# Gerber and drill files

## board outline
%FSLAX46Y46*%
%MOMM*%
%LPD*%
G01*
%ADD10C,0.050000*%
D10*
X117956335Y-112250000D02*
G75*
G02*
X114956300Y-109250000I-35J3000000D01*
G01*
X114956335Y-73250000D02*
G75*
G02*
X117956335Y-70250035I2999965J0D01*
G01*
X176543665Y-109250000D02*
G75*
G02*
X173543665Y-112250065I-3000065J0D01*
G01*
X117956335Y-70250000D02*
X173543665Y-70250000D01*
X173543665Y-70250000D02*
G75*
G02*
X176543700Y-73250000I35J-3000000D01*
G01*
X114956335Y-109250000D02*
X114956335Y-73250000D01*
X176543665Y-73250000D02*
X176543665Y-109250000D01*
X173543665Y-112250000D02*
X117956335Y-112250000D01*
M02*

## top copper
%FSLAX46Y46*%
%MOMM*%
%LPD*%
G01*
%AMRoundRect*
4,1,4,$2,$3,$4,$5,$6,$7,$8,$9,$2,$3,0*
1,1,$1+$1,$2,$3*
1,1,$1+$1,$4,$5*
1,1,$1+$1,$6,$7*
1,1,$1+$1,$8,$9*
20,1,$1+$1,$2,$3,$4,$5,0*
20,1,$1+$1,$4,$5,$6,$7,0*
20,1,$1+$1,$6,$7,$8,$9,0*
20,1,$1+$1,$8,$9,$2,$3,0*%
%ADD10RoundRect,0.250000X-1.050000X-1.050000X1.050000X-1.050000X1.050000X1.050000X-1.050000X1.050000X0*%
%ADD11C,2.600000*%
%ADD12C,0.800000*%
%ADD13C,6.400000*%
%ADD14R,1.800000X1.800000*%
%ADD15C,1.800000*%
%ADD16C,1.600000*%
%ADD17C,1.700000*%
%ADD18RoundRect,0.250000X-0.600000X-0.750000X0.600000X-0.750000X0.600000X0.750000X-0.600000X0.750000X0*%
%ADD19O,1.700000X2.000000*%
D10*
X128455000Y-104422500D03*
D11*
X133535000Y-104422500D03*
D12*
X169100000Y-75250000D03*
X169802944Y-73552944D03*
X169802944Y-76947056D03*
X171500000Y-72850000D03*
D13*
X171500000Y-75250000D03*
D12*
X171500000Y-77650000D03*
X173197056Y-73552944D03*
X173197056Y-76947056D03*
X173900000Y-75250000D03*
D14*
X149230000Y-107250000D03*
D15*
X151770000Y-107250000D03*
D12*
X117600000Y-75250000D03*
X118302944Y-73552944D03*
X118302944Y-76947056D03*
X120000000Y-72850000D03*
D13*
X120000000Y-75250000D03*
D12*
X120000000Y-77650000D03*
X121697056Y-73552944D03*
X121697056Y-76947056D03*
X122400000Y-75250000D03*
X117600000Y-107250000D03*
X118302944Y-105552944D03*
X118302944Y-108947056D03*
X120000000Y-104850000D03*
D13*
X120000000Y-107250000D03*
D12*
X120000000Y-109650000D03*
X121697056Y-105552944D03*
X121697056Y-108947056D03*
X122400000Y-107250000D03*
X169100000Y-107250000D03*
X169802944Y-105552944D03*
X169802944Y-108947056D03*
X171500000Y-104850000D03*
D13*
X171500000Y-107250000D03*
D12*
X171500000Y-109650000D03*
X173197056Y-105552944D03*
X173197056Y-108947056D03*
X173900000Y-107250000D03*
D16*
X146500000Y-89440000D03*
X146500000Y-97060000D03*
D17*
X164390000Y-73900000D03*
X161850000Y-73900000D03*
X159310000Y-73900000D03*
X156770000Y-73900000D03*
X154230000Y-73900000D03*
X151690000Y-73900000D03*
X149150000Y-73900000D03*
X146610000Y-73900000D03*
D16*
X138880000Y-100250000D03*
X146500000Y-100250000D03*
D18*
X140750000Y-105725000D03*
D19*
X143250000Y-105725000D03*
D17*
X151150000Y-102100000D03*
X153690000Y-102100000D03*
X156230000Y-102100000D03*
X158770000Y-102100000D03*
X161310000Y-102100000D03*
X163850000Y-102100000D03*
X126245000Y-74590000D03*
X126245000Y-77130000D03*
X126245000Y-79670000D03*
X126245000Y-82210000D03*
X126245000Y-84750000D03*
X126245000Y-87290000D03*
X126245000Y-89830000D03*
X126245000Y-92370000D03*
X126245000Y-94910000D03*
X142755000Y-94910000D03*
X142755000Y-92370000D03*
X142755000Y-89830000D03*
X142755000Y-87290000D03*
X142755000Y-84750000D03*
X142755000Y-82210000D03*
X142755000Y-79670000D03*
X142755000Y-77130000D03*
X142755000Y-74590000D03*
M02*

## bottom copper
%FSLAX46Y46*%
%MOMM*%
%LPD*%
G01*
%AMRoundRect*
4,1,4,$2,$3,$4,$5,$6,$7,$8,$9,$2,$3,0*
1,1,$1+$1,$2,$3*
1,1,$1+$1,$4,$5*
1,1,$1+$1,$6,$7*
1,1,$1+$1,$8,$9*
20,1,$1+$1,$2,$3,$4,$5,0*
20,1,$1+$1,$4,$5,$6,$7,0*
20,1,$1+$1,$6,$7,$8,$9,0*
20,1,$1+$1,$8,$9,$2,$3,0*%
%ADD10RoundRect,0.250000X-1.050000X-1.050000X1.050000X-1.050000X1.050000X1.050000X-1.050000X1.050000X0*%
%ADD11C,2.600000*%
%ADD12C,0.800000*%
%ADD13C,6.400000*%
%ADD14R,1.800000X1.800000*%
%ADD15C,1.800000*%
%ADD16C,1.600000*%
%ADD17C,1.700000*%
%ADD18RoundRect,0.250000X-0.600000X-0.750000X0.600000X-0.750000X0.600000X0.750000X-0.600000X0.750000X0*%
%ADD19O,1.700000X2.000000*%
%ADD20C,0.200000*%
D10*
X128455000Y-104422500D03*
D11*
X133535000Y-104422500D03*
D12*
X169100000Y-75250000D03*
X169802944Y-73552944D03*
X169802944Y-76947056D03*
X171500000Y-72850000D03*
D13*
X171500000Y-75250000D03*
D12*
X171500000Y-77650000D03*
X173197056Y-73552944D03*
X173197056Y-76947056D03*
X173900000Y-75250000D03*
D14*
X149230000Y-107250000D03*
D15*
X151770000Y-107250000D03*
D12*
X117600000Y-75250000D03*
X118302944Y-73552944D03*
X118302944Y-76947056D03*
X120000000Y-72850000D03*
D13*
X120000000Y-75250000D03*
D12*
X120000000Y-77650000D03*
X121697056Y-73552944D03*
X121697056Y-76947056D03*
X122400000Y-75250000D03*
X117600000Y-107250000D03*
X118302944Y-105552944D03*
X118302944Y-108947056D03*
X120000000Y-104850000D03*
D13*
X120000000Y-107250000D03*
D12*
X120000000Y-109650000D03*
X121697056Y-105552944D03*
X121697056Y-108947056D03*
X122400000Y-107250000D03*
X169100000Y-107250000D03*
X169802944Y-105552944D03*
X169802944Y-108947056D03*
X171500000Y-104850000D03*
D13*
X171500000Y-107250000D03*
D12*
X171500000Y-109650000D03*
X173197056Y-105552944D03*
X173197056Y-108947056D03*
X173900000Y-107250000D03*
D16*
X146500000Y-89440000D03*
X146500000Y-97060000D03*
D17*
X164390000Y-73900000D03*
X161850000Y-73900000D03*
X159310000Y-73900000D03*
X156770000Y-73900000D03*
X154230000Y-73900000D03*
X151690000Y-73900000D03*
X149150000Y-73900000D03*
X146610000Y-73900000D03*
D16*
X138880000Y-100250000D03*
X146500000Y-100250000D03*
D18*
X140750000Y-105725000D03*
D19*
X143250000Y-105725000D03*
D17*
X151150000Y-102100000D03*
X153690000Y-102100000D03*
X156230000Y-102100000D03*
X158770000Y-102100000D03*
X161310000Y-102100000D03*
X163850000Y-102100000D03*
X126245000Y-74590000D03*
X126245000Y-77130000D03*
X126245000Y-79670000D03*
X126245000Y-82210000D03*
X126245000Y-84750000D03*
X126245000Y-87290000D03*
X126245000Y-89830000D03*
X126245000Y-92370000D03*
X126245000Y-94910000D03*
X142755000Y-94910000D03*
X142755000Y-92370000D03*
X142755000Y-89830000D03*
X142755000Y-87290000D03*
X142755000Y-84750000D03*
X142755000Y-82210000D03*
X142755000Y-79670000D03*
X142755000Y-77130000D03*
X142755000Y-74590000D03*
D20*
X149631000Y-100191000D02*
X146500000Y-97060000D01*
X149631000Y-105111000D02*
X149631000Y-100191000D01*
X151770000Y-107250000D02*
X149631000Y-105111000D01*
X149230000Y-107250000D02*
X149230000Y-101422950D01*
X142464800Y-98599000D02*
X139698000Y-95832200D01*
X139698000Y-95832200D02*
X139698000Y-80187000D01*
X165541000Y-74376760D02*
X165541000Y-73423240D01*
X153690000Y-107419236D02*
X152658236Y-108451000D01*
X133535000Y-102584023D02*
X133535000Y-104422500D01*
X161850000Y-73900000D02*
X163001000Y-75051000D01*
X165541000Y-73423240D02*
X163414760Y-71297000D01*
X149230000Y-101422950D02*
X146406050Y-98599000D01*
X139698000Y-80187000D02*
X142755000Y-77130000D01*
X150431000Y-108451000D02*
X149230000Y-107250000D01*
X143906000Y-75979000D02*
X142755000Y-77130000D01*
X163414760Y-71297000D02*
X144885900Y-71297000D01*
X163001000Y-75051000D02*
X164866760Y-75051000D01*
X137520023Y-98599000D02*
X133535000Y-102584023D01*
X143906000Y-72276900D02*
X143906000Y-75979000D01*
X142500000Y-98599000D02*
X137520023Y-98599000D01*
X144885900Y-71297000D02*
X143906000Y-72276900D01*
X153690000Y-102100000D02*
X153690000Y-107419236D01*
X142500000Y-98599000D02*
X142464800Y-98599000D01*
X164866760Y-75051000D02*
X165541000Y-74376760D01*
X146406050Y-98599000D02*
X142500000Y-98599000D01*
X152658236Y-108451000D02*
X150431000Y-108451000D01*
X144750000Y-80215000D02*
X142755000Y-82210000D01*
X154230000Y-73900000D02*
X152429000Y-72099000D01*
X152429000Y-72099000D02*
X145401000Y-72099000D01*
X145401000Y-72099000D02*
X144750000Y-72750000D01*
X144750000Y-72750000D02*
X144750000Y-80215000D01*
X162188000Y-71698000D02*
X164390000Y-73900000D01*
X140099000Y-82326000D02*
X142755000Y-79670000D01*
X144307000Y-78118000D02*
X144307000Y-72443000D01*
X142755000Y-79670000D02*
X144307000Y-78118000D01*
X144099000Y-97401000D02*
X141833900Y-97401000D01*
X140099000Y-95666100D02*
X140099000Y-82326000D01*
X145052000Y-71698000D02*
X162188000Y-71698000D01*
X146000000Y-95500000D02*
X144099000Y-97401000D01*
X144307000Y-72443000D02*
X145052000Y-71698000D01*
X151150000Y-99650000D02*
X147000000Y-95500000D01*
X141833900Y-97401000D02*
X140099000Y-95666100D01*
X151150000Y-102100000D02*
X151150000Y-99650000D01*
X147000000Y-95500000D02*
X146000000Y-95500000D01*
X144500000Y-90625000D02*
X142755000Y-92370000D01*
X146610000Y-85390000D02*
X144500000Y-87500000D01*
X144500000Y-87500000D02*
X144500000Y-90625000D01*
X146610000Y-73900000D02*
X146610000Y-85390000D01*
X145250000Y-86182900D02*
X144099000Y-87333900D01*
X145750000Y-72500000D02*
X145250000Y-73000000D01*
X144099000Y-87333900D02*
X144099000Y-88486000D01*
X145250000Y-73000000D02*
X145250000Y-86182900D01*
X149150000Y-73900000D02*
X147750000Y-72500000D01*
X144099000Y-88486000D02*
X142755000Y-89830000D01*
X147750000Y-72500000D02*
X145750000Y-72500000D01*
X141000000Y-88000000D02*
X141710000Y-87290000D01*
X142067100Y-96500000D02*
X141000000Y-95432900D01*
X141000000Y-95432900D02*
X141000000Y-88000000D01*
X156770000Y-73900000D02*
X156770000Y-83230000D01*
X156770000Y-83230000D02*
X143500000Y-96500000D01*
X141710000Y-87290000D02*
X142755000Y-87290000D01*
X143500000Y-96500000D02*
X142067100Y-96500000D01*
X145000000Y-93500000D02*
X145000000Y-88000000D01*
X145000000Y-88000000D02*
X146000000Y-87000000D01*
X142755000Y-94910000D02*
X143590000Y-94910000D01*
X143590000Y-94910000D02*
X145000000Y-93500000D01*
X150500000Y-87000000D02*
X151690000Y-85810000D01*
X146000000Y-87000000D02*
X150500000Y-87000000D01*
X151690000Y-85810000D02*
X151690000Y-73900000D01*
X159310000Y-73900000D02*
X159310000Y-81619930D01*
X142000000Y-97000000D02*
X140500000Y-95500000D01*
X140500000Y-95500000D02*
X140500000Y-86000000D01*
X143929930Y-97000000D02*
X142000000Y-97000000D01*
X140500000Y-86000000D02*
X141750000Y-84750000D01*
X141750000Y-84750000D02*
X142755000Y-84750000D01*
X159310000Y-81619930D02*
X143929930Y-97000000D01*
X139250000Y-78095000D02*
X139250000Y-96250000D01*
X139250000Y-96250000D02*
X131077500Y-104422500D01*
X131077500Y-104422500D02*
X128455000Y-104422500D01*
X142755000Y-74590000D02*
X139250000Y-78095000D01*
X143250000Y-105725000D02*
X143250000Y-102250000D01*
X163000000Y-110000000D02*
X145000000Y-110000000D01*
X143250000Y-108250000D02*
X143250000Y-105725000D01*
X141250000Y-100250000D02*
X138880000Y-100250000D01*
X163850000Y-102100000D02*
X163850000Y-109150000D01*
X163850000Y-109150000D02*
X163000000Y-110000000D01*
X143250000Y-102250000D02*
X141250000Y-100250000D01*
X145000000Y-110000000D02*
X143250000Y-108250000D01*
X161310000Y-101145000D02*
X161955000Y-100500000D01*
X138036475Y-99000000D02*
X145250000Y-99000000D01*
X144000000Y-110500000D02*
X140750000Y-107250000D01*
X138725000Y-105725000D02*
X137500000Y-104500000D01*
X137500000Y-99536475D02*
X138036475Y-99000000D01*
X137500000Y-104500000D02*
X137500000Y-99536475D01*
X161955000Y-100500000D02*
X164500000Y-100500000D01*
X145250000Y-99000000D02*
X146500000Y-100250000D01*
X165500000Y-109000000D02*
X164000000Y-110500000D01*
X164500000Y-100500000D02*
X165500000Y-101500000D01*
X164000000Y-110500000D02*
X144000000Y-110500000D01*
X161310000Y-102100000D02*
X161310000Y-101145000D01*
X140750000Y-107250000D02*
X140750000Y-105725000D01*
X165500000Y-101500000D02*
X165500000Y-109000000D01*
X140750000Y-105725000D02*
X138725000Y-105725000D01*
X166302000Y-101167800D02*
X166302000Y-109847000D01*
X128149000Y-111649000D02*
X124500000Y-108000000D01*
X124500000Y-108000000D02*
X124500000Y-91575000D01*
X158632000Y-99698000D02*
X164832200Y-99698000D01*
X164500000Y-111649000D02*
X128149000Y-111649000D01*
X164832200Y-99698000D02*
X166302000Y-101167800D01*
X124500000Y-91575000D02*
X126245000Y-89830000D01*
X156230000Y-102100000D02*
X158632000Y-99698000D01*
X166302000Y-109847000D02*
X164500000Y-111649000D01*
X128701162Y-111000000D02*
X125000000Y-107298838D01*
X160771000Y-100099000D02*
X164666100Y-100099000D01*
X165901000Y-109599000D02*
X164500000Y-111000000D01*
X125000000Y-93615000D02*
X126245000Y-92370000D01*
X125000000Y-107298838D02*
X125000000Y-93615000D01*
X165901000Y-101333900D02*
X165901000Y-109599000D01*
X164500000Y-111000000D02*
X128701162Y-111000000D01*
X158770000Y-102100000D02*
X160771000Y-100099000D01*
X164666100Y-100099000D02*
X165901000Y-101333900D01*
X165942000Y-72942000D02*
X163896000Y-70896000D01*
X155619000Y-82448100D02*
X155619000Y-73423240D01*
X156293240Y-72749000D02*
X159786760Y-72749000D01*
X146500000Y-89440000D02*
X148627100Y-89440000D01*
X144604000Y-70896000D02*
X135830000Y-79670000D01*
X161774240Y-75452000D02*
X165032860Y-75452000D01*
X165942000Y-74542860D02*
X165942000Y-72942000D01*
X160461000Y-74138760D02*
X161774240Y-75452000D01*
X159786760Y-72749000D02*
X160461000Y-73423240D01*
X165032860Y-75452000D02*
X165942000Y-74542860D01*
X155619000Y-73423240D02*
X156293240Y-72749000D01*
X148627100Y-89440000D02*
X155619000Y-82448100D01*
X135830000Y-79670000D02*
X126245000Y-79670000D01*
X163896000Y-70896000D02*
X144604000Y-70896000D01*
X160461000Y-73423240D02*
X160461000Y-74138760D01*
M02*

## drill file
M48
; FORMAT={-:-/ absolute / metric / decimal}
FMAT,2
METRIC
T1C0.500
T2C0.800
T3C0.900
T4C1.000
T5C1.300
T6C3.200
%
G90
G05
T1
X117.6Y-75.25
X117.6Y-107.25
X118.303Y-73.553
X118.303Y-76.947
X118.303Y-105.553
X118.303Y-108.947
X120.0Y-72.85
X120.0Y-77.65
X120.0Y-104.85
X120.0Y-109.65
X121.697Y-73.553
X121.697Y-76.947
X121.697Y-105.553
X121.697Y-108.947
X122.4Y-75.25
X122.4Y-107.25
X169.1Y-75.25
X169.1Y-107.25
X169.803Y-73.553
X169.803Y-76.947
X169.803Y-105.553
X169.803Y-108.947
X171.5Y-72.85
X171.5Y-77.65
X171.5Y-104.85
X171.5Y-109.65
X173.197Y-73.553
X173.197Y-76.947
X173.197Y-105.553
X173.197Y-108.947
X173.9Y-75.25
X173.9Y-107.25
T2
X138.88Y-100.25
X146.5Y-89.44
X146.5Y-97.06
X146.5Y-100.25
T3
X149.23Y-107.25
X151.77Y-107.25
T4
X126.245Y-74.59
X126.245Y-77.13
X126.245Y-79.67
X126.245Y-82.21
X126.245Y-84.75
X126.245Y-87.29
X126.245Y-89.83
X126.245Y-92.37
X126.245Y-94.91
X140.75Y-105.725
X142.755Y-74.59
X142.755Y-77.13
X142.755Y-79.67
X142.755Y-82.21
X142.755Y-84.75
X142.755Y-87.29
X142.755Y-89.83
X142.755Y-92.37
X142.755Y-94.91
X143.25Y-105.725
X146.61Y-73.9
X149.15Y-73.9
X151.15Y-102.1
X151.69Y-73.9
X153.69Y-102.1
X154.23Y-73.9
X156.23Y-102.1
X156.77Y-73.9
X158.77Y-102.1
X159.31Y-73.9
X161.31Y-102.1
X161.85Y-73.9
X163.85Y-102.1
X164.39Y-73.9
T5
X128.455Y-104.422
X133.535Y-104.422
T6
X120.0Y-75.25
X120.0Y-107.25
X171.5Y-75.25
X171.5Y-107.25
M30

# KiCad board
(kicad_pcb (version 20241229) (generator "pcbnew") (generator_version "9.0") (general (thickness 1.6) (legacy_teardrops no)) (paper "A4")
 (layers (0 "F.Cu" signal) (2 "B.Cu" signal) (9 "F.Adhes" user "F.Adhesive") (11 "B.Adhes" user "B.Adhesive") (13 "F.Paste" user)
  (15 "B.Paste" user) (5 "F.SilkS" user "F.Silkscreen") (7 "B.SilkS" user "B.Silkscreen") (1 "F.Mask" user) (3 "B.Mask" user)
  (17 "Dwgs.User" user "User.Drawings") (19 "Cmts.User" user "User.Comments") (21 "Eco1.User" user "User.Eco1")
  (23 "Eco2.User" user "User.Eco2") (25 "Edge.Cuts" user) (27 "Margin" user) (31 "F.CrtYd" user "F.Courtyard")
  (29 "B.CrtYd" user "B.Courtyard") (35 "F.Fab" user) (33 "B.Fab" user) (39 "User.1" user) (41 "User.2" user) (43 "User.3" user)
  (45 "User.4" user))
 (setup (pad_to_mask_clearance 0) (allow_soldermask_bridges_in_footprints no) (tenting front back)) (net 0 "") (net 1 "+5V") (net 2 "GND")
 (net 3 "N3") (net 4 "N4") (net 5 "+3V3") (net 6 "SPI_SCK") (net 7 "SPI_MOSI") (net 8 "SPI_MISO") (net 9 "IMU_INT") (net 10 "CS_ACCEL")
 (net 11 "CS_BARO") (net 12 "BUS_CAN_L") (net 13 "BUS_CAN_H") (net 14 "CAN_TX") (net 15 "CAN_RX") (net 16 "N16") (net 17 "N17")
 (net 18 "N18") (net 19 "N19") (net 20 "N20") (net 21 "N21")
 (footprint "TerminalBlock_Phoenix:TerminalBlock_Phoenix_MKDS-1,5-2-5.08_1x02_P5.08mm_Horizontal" (layer "F.Cu") (at 128.455 104.4225)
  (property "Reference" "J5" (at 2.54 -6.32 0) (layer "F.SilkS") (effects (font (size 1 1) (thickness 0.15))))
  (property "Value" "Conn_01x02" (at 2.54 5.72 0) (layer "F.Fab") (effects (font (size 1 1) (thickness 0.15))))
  (pad "1" thru_hole roundrect (at 0 0) (size 2.6 2.6) (drill 1.3) (layers "*.Cu" "*.Mask") (remove_unused_layers no)
   (roundrect_rratio 0.096154) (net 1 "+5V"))
  (pad "2" thru_hole circle (at 5.08 0) (size 2.6 2.6) (drill 1.3) (layers "*.Cu" "*.Mask") (remove_unused_layers no) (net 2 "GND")))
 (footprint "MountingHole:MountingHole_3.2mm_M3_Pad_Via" (layer "F.Cu") (at 171.5 75.25)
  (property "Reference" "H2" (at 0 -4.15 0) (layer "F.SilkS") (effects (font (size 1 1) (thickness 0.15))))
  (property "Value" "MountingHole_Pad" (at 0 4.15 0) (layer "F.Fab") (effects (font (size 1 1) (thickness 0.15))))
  (pad "1" thru_hole circle (at -2.4 0) (size 0.8 0.8) (drill 0.5) (layers "*.Cu" "*.Mask") (remove_unused_layers no) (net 2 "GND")
   (zone_connect 2))
  (pad "1" thru_hole circle (at -1.697056 -1.697056) (size 0.8 0.8) (drill 0.5) (layers "*.Cu" "*.Mask") (remove_unused_layers no)
   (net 2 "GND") (zone_connect 2))
  (pad "1" thru_hole circle (at -1.697056 1.697056) (size 0.8 0.8) (drill 0.5) (layers "*.Cu" "*.Mask") (remove_unused_layers no)
   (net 2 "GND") (zone_connect 2))
  (pad "1" thru_hole circle (at 0 -2.4) (size 0.8 0.8) (drill 0.5) (layers "*.Cu" "*.Mask") (remove_unused_layers no) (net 2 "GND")
   (zone_connect 2))
  (pad "1" thru_hole circle (at 0 0) (size 6.4 6.4) (drill 3.2) (layers "*.Cu" "*.Mask") (remove_unused_layers no) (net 2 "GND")
   (zone_connect 2))
  (pad "1" thru_hole circle (at 0 2.4) (size 0.8 0.8) (drill 0.5) (layers "*.Cu" "*.Mask") (remove_unused_layers no) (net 2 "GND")
   (zone_connect 2))
  (pad "1" thru_hole circle (at 1.697056 -1.697056) (size 0.8 0.8) (drill 0.5) (layers "*.Cu" "*.Mask") (remove_unused_layers no)
   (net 2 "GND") (zone_connect 2))
  (pad "1" thru_hole circle (at 1.697056 1.697056) (size 0.8 0.8) (drill 0.5) (layers "*.Cu" "*.Mask") (remove_unused_layers no)
   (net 2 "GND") (zone_connect 2))
  (pad "1" thru_hole circle (at 2.4 0) (size 0.8 0.8) (drill 0.5) (layers "*.Cu" "*.Mask") (remove_unused_layers no) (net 2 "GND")
   (zone_connect 2)))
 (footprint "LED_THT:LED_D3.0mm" (layer "F.Cu") (at 149.23 107.25)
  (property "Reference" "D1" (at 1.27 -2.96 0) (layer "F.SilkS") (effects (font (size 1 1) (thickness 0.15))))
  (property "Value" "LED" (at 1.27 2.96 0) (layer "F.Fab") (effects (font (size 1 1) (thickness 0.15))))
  (pad "1" thru_hole rect (at 0 0) (size 1.8 1.8) (drill 0.9) (layers "*.Cu" "*.Mask") (remove_unused_layers no) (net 2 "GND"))
  (pad "2" thru_hole circle (at 2.54 0) (size 1.8 1.8) (drill 0.9) (layers "*.Cu" "*.Mask") (remove_unused_layers no) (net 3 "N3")))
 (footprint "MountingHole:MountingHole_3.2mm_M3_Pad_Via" (layer "F.Cu") (at 120 75.25)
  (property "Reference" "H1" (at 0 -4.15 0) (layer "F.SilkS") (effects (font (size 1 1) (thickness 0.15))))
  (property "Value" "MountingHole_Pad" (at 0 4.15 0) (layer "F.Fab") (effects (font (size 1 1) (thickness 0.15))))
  (pad "1" thru_hole circle (at -2.4 0) (size 0.8 0.8) (drill 0.5) (layers "*.Cu" "*.Mask") (remove_unused_layers no) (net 2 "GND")
   (zone_connect 2))
  (pad "1" thru_hole circle (at -1.697056 -1.697056) (size 0.8 0.8) (drill 0.5) (layers "*.Cu" "*.Mask") (remove_unused_layers no)
   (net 2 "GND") (zone_connect 2))
  (pad "1" thru_hole circle (at -1.697056 1.697056) (size 0.8 0.8) (drill 0.5) (layers "*.Cu" "*.Mask") (remove_unused_layers no)
   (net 2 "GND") (zone_connect 2))
  (pad "1" thru_hole circle (at 0 -2.4) (size 0.8 0.8) (drill 0.5) (layers "*.Cu" "*.Mask") (remove_unused_layers no) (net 2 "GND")
   (zone_connect 2))
  (pad "1" thru_hole circle (at 0 0) (size 6.4 6.4) (drill 3.2) (layers "*.Cu" "*.Mask") (remove_unused_layers no) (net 2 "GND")
   (zone_connect 2))
  (pad "1" thru_hole circle (at 0 2.4) (size 0.8 0.8) (drill 0.5) (layers "*.Cu" "*.Mask") (remove_unused_layers no) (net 2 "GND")
   (zone_connect 2))
  (pad "1" thru_hole circle (at 1.697056 -1.697056) (size 0.8 0.8) (drill 0.5) (layers "*.Cu" "*.Mask") (remove_unused_layers no)
   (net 2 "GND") (zone_connect 2))
  (pad "1" thru_hole circle (at 1.697056 1.697056) (size 0.8 0.8) (drill 0.5) (layers "*.Cu" "*.Mask") (remove_unused_layers no)
   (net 2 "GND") (zone_connect 2))
  (pad "1" thru_hole circle (at 2.4 0) (size 0.8 0.8) (drill 0.5) (layers "*.Cu" "*.Mask") (remove_unused_layers no) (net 2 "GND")
   (zone_connect 2)))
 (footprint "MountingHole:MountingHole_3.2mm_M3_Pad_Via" (layer "F.Cu") (at 120 107.25)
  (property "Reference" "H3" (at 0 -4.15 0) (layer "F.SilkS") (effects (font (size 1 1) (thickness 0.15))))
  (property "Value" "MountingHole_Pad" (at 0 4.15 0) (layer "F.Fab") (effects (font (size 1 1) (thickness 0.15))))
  (pad "1" thru_hole circle (at -2.4 0) (size 0.8 0.8) (drill 0.5) (layers "*.Cu" "*.Mask") (remove_unused_layers no) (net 2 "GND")
   (zone_connect 2))
  (pad "1" thru_hole circle (at -1.697056 -1.697056) (size 0.8 0.8) (drill 0.5) (layers "*.Cu" "*.Mask") (remove_unused_layers no)
   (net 2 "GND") (zone_connect 2))
  (pad "1" thru_hole circle (at -1.697056 1.697056) (size 0.8 0.8) (drill 0.5) (layers "*.Cu" "*.Mask") (remove_unused_layers no)
   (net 2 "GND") (zone_connect 2))
  (pad "1" thru_hole circle (at 0 -2.4) (size 0.8 0.8) (drill 0.5) (layers "*.Cu" "*.Mask") (remove_unused_layers no) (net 2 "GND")
   (zone_connect 2))
  (pad "1" thru_hole circle (at 0 0) (size 6.4 6.4) (drill 3.2) (layers "*.Cu" "*.Mask") (remove_unused_layers no) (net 2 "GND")
   (zone_connect 2))
  (pad "1" thru_hole circle (at 0 2.4) (size 0.8 0.8) (drill 0.5) (layers "*.Cu" "*.Mask") (remove_unused_layers no) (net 2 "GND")
   (zone_connect 2))
  (pad "1" thru_hole circle (at 1.697056 -1.697056) (size 0.8 0.8) (drill 0.5) (layers "*.Cu" "*.Mask") (remove_unused_layers no)
   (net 2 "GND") (zone_connect 2))
  (pad "1" thru_hole circle (at 1.697056 1.697056) (size 0.8 0.8) (drill 0.5) (layers "*.Cu" "*.Mask") (remove_unused_layers no)
   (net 2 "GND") (zone_connect 2))
  (pad "1" thru_hole circle (at 2.4 0) (size 0.8 0.8) (drill 0.5) (layers "*.Cu" "*.Mask") (remove_unused_layers no) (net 2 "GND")
   (zone_connect 2)))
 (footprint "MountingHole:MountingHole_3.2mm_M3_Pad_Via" (layer "F.Cu") (at 171.5 107.25)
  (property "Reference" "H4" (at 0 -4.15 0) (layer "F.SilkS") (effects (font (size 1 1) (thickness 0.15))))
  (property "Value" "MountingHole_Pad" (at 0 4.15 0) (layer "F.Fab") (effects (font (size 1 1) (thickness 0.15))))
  (pad "1" thru_hole circle (at -2.4 0) (size 0.8 0.8) (drill 0.5) (layers "*.Cu" "*.Mask") (remove_unused_layers no) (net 2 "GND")
   (zone_connect 2))
  (pad "1" thru_hole circle (at -1.697056 -1.697056) (size 0.8 0.8) (drill 0.5) (layers "*.Cu" "*.Mask") (remove_unused_layers no)
   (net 2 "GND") (zone_connect 2))
  (pad "1" thru_hole circle (at -1.697056 1.697056) (size 0.8 0.8) (drill 0.5) (layers "*.Cu" "*.Mask") (remove_unused_layers no)
   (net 2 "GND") (zone_connect 2))
  (pad "1" thru_hole circle (at 0 -2.4) (size 0.8 0.8) (drill 0.5) (layers "*.Cu" "*.Mask") (remove_unused_layers no) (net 2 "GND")
   (zone_connect 2))
  (pad "1" thru_hole circle (at 0 0) (size 6.4 6.4) (drill 3.2) (layers "*.Cu" "*.Mask") (remove_unused_layers no) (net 2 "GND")
   (zone_connect 2))
  (pad "1" thru_hole circle (at 0 2.4) (size 0.8 0.8) (drill 0.5) (layers "*.Cu" "*.Mask") (remove_unused_layers no) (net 2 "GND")
   (zone_connect 2))
  (pad "1" thru_hole circle (at 1.697056 -1.697056) (size 0.8 0.8) (drill 0.5) (layers "*.Cu" "*.Mask") (remove_unused_layers no)
   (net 2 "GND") (zone_connect 2))
  (pad "1" thru_hole circle (at 1.697056 1.697056) (size 0.8 0.8) (drill 0.5) (layers "*.Cu" "*.Mask") (remove_unused_layers no)
   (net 2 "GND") (zone_connect 2))
  (pad "1" thru_hole circle (at 2.4 0) (size 0.8 0.8) (drill 0.5) (layers "*.Cu" "*.Mask") (remove_unused_layers no) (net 2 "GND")
   (zone_connect 2)))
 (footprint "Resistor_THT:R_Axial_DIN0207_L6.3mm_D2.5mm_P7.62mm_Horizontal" (layer "F.Cu") (at 146.5 89.44 -90)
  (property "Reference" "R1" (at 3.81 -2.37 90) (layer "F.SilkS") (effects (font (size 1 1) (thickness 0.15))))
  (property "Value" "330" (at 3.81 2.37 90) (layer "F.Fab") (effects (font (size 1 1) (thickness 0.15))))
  (pad "1" thru_hole circle (at 0 0 270) (size 1.6 1.6) (drill 0.8) (layers "*.Cu" "*.Mask") (remove_unused_layers no) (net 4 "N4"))
  (pad "2" thru_hole circle (at 7.62 0 270) (size 1.6 1.6) (drill 0.8) (layers "*.Cu" "*.Mask") (remove_unused_layers no) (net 3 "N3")))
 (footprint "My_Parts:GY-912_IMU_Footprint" (layer "F.Cu") (at 155.5 80.25 -90)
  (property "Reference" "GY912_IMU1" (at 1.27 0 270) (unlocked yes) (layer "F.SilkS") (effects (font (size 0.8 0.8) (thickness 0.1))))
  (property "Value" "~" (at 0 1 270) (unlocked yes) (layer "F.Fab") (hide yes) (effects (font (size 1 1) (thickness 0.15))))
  (pad "1" thru_hole circle (at -6.35 -8.89 270) (size 1.7 1.7) (drill 1) (layers "*.Cu" "*.Mask") (remove_unused_layers no) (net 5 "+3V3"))
  (pad "2" thru_hole circle (at -6.35 -6.35 270) (size 1.7 1.7) (drill 1) (layers "*.Cu" "*.Mask") (remove_unused_layers no) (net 2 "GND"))
  (pad "3" thru_hole circle (at -6.35 -3.81 270) (size 1.7 1.7) (drill 1) (layers "*.Cu" "*.Mask") (remove_unused_layers no)
   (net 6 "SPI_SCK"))
  (pad "4" thru_hole circle (at -6.35 -1.27 270) (size 1.7 1.7) (drill 1) (layers "*.Cu" "*.Mask") (remove_unused_layers no)
   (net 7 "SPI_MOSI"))
  (pad "5" thru_hole circle (at -6.35 1.27 270) (size 1.7 1.7) (drill 1) (layers "*.Cu" "*.Mask") (remove_unused_layers no)
   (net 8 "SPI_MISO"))
  (pad "6" thru_hole circle (at -6.35 3.81 270) (size 1.7 1.7) (drill 1) (layers "*.Cu" "*.Mask") (remove_unused_layers no)
   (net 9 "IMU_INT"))
  (pad "7" thru_hole circle (at -6.35 6.35 270) (size 1.7 1.7) (drill 1) (layers "*.Cu" "*.Mask") (remove_unused_layers no)
   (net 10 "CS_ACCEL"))
  (pad "8" thru_hole circle (at -6.35 8.89 270) (size 1.7 1.7) (drill 1) (layers "*.Cu" "*.Mask") (remove_unused_layers no)
   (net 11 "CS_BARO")))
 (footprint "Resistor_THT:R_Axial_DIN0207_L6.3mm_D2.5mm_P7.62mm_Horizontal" (layer "F.Cu") (at 138.88 100.25)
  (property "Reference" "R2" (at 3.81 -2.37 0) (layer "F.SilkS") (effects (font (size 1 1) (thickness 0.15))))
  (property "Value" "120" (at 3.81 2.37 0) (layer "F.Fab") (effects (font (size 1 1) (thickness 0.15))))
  (pad "1" thru_hole circle (at 0 0) (size 1.6 1.6) (drill 0.8) (layers "*.Cu" "*.Mask") (remove_unused_layers no) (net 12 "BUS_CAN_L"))
  (pad "2" thru_hole circle (at 7.62 0) (size 1.6 1.6) (drill 0.8) (layers "*.Cu" "*.Mask") (remove_unused_layers no) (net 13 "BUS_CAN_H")))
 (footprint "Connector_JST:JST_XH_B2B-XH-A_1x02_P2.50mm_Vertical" (layer "F.Cu") (at 140.75 105.725)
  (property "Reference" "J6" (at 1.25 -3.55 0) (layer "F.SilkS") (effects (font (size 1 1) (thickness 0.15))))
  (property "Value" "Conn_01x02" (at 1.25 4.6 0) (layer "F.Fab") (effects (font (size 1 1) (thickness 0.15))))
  (pad "1" thru_hole roundrect (at 0 0) (size 1.7 2) (drill 1) (layers "*.Cu" "*.Mask") (remove_unused_layers no)
   (roundrect_rratio 0.147059) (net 13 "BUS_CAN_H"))
  (pad "2" thru_hole oval (at 2.5 0) (size 1.7 2) (drill 1) (layers "*.Cu" "*.Mask") (remove_unused_layers no) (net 12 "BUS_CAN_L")))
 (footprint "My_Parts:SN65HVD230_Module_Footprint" (layer "F.Cu") (at 157.5 95.75 90)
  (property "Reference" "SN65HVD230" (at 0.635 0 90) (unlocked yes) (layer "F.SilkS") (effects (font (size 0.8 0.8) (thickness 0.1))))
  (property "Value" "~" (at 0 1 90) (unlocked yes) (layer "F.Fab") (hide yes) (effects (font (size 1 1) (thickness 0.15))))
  (pad "1" thru_hole circle (at -6.35 -6.35 90) (size 1.7 1.7) (drill 1) (layers "*.Cu" "*.Mask") (remove_unused_layers no) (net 5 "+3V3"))
  (pad "2" thru_hole circle (at -6.35 -3.81 90) (size 1.7 1.7) (drill 1) (layers "*.Cu" "*.Mask") (remove_unused_layers no) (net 2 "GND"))
  (pad "3" thru_hole circle (at -6.35 -1.27 90) (size 1.7 1.7) (drill 1) (layers "*.Cu" "*.Mask") (remove_unused_layers no)
   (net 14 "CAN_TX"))
  (pad "4" thru_hole circle (at -6.35 1.27 90) (size 1.7 1.7) (drill 1) (layers "*.Cu" "*.Mask") (remove_unused_layers no) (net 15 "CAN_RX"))
  (pad "5" thru_hole circle (at -6.35 3.81 90) (size 1.7 1.7) (drill 1) (layers "*.Cu" "*.Mask") (remove_unused_layers no)
   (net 13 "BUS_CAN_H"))
  (pad "6" thru_hole circle (at -6.35 6.35 90) (size 1.7 1.7) (drill 1) (layers "*.Cu" "*.Mask") (remove_unused_layers no)
   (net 12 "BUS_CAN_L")))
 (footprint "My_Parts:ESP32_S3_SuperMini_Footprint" (layer "F.Cu") (at 134.5 84.75)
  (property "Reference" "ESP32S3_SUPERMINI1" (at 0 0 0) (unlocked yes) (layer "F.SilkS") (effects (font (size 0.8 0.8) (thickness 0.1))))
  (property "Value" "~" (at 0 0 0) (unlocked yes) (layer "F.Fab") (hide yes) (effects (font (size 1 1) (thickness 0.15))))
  (pad "1" thru_hole circle (at -8.255 -10.16) (size 1.7 1.7) (drill 1) (layers "*.Cu" "*.Mask") (remove_unused_layers no) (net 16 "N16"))
  (pad "2" thru_hole circle (at -8.255 -7.62) (size 1.7 1.7) (drill 1) (layers "*.Cu" "*.Mask") (remove_unused_layers no) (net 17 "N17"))
  (pad "3" thru_hole circle (at -8.255 -5.08) (size 1.7 1.7) (drill 1) (layers "*.Cu" "*.Mask") (remove_unused_layers no) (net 4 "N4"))
  (pad "4" thru_hole circle (at -8.255 -2.54) (size 1.7 1.7) (drill 1) (layers "*.Cu" "*.Mask") (remove_unused_layers no) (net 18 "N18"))
  (pad "5" thru_hole circle (at -8.255 0) (size 1.7 1.7) (drill 1) (layers "*.Cu" "*.Mask") (remove_unused_layers no) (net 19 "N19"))
  (pad "6" thru_hole circle (at -8.255 2.54) (size 1.7 1.7) (drill 1) (layers "*.Cu" "*.Mask") (remove_unused_layers no) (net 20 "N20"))
  (pad "7" thru_hole circle (at -8.255 5.08) (size 1.7 1.7) (drill 1) (layers "*.Cu" "*.Mask") (remove_unused_layers no) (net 14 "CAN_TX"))
  (pad "8" thru_hole circle (at -8.255 7.62) (size 1.7 1.7) (drill 1) (layers "*.Cu" "*.Mask") (remove_unused_layers no) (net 15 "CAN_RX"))
  (pad "9" thru_hole circle (at -8.255 10.16) (size 1.7 1.7) (drill 1) (layers "*.Cu" "*.Mask") (remove_unused_layers no) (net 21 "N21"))
  (pad "10" thru_hole circle (at 8.255 10.16) (size 1.7 1.7) (drill 1) (layers "*.Cu" "*.Mask") (remove_unused_layers no) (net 9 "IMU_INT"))
  (pad "11" thru_hole circle (at 8.255 7.62) (size 1.7 1.7) (drill 1) (layers "*.Cu" "*.Mask") (remove_unused_layers no) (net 11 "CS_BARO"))
  (pad "12" thru_hole circle (at 8.255 5.08) (size 1.7 1.7) (drill 1) (layers "*.Cu" "*.Mask") (remove_unused_layers no) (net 10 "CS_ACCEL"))
  (pad "13" thru_hole circle (at 8.255 2.54) (size 1.7 1.7) (drill 1) (layers "*.Cu" "*.Mask") (remove_unused_layers no) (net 7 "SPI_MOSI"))
  (pad "14" thru_hole circle (at 8.255 0) (size 1.7 1.7) (drill 1) (layers "*.Cu" "*.Mask") (remove_unused_layers no) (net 6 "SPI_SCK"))
  (pad "15" thru_hole circle (at 8.255 -2.54) (size 1.7 1.7) (drill 1) (layers "*.Cu" "*.Mask") (remove_unused_layers no) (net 8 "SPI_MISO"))
  (pad "16" thru_hole circle (at 8.255 -5.08) (size 1.7 1.7) (drill 1) (layers "*.Cu" "*.Mask") (remove_unused_layers no) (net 5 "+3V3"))
  (pad "17" thru_hole circle (at 8.255 -7.62) (size 1.7 1.7) (drill 1) (layers "*.Cu" "*.Mask") (remove_unused_layers no) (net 2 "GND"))
  (pad "18" thru_hole circle (at 8.255 -10.16) (size 1.7 1.7) (drill 1) (layers "*.Cu" "*.Mask") (remove_unused_layers no) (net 1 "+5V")))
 (gr_arc (start 117.956335 112.25) (mid 115.835015 111.37132) (end 114.956335 109.25) (stroke (width 0.05) (type default))
  (layer "Edge.Cuts"))
 (gr_arc (start 114.956335 73.25) (mid 115.835015 71.12868) (end 117.956335 70.25) (stroke (width 0.05) (type default)) (layer "Edge.Cuts"))
 (gr_arc (start 176.543665 109.25) (mid 175.664983 111.371308) (end 173.543665 112.25) (stroke (width 0.05) (type default))
  (layer "Edge.Cuts"))
 (gr_line (start 117.956335 70.25) (end 173.543665 70.25) (stroke (width 0.05) (type default)) (layer "Edge.Cuts"))
 (gr_arc (start 173.543665 70.25) (mid 175.664985 71.12868) (end 176.543665 73.25) (stroke (width 0.05) (type default)) (layer "Edge.Cuts"))
 (gr_line (start 114.956335 109.25) (end 114.956335 73.25) (stroke (width 0.05) (type default)) (layer "Edge.Cuts"))
 (gr_line (start 176.543665 73.25) (end 176.543665 109.25) (stroke (width 0.05) (type default)) (layer "Edge.Cuts"))
 (gr_line (start 173.543665 112.25) (end 117.956335 112.25) (stroke (width 0.05) (type default)) (layer "Edge.Cuts"))
 (segment (start 149.631 100.191) (end 146.5 97.06) (width 0.2) (layer "B.Cu") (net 3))
 (segment (start 149.631 105.111) (end 149.631 100.191) (width 0.2) (layer "B.Cu") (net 3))
 (segment (start 151.77 107.25) (end 149.631 105.111) (width 0.2) (layer "B.Cu") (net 3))
 (segment (start 149.23 107.25) (end 149.23 101.42295) (width 0.2) (layer "B.Cu") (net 2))
 (segment (start 142.4648 98.599) (end 139.698 95.8322) (width 0.2) (layer "B.Cu") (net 2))
 (segment (start 139.698 95.8322) (end 139.698 80.187) (width 0.2) (layer "B.Cu") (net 2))
 (segment (start 165.541 74.37676) (end 165.541 73.42324) (width 0.2) (layer "B.Cu") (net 2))
 (segment (start 153.69 107.419236) (end 152.658236 108.451) (width 0.2) (layer "B.Cu") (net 2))
 (segment (start 133.535 102.584023) (end 133.535 104.4225) (width 0.2) (layer "B.Cu") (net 2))
 (segment (start 161.85 73.9) (end 163.001 75.051) (width 0.2) (layer "B.Cu") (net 2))
 (segment (start 165.541 73.42324) (end 163.41476 71.297) (width 0.2) (layer "B.Cu") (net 2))
 (segment (start 149.23 101.42295) (end 146.40605 98.599) (width 0.2) (layer "B.Cu") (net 2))
 (segment (start 139.698 80.187) (end 142.755 77.13) (width 0.2) (layer "B.Cu") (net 2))
 (segment (start 150.431 108.451) (end 149.23 107.25) (width 0.2) (layer "B.Cu") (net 2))
 (segment (start 143.906 75.979) (end 142.755 77.13) (width 0.2) (layer "B.Cu") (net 2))
 (segment (start 163.41476 71.297) (end 144.8859 71.297) (width 0.2) (layer "B.Cu") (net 2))
 (segment (start 163.001 75.051) (end 164.86676 75.051) (width 0.2) (layer "B.Cu") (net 2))
 (segment (start 137.520023 98.599) (end 133.535 102.584023) (width 0.2) (layer "B.Cu") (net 2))
 (segment (start 143.906 72.2769) (end 143.906 75.979) (width 0.2) (layer "B.Cu") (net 2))
 (segment (start 142.5 98.599) (end 137.520023 98.599) (width 0.2) (layer "B.Cu") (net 2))
 (segment (start 144.8859 71.297) (end 143.906 72.2769) (width 0.2) (layer "B.Cu") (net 2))
 (segment (start 153.69 102.1) (end 153.69 107.419236) (width 0.2) (layer "B.Cu") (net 2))
 (segment (start 142.5 98.599) (end 142.4648 98.599) (width 0.2) (layer "B.Cu") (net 2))
 (segment (start 164.86676 75.051) (end 165.541 74.37676) (width 0.2) (layer "B.Cu") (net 2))
 (segment (start 146.40605 98.599) (end 142.5 98.599) (width 0.2) (layer "B.Cu") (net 2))
 (segment (start 152.658236 108.451) (end 150.431 108.451) (width 0.2) (layer "B.Cu") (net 2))
 (segment (start 144.75 80.215) (end 142.755 82.21) (width 0.2) (layer "B.Cu") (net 8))
 (segment (start 154.23 73.9) (end 152.429 72.099) (width 0.2) (layer "B.Cu") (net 8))
 (segment (start 152.429 72.099) (end 145.401 72.099) (width 0.2) (layer "B.Cu") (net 8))
 (segment (start 145.401 72.099) (end 144.75 72.75) (width 0.2) (layer "B.Cu") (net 8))
 (segment (start 144.75 72.75) (end 144.75 80.215) (width 0.2) (layer "B.Cu") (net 8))
 (segment (start 162.188 71.698) (end 164.39 73.9) (width 0.2) (layer "B.Cu") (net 5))
 (segment (start 140.099 82.326) (end 142.755 79.67) (width 0.2) (layer "B.Cu") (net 5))
 (segment (start 144.307 78.118) (end 144.307 72.443) (width 0.2) (layer "B.Cu") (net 5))
 (segment (start 142.755 79.67) (end 144.307 78.118) (width 0.2) (layer "B.Cu") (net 5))
 (segment (start 144.099 97.401) (end 141.8339 97.401) (width 0.2) (layer "B.Cu") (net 5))
 (segment (start 140.099 95.6661) (end 140.099 82.326) (width 0.2) (layer "B.Cu") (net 5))
 (segment (start 145.052 71.698) (end 162.188 71.698) (width 0.2) (layer "B.Cu") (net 5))
 (segment (start 146 95.5) (end 144.099 97.401) (width 0.2) (layer "B.Cu") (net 5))
 (segment (start 144.307 72.443) (end 145.052 71.698) (width 0.2) (layer "B.Cu") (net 5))
 (segment (start 151.15 99.65) (end 147 95.5) (width 0.2) (layer "B.Cu") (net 5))
 (segment (start 141.8339 97.401) (end 140.099 95.6661) (width 0.2) (layer "B.Cu") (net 5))
 (segment (start 151.15 102.1) (end 151.15 99.65) (width 0.2) (layer "B.Cu") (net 5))
 (segment (start 147 95.5) (end 146 95.5) (width 0.2) (layer "B.Cu") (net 5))
 (segment (start 144.5 90.625) (end 142.755 92.37) (width 0.2) (layer "B.Cu") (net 11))
 (segment (start 146.61 85.39) (end 144.5 87.5) (width 0.2) (layer "B.Cu") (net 11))
 (segment (start 144.5 87.5) (end 144.5 90.625) (width 0.2) (layer "B.Cu") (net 11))
 (segment (start 146.61 73.9) (end 146.61 85.39) (width 0.2) (layer "B.Cu") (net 11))
 (segment (start 145.25 86.1829) (end 144.099 87.3339) (width 0.2) (layer "B.Cu") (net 10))
 (segment (start 145.75 72.5) (end 145.25 73) (width 0.2) (layer "B.Cu") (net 10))
 (segment (start 144.099 87.3339) (end 144.099 88.486) (width 0.2) (layer "B.Cu") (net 10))
 (segment (start 145.25 73) (end 145.25 86.1829) (width 0.2) (layer "B.Cu") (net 10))
 (segment (start 149.15 73.9) (end 147.75 72.5) (width 0.2) (layer "B.Cu") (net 10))
 (segment (start 144.099 88.486) (end 142.755 89.83) (width 0.2) (layer "B.Cu") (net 10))
 (segment (start 147.75 72.5) (end 145.75 72.5) (width 0.2) (layer "B.Cu") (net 10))
 (segment (start 141 88) (end 141.71 87.29) (width 0.2) (layer "B.Cu") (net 7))
 (segment (start 142.0671 96.5) (end 141 95.4329) (width 0.2) (layer "B.Cu") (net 7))
 (segment (start 141 95.4329) (end 141 88) (width 0.2) (layer "B.Cu") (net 7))
 (segment (start 156.77 73.9) (end 156.77 83.23) (width 0.2) (layer "B.Cu") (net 7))
 (segment (start 156.77 83.23) (end 143.5 96.5) (width 0.2) (layer "B.Cu") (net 7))
 (segment (start 141.71 87.29) (end 142.755 87.29) (width 0.2) (layer "B.Cu") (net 7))
 (segment (start 143.5 96.5) (end 142.0671 96.5) (width 0.2) (layer "B.Cu") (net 7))
 (segment (start 145 93.5) (end 145 88) (width 0.2) (layer "B.Cu") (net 9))
 (segment (start 145 88) (end 146 87) (width 0.2) (layer "B.Cu") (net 9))
 (segment (start 142.755 94.91) (end 143.59 94.91) (width 0.2) (layer "B.Cu") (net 9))
 (segment (start 143.59 94.91) (end 145 93.5) (width 0.2) (layer "B.Cu") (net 9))
 (segment (start 150.5 87) (end 151.69 85.81) (width 0.2) (layer "B.Cu") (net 9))
 (segment (start 146 87) (end 150.5 87) (width 0.2) (layer "B.Cu") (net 9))
 (segment (start 151.69 85.81) (end 151.69 73.9) (width 0.2) (layer "B.Cu") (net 9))
 (segment (start 159.31 73.9) (end 159.31 81.61993) (width 0.2) (layer "B.Cu") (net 6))
 (segment (start 142 97) (end 140.5 95.5) (width 0.2) (layer "B.Cu") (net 6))
 (segment (start 140.5 95.5) (end 140.5 86) (width 0.2) (layer "B.Cu") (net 6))
 (segment (start 143.92993 97) (end 142 97) (width 0.2) (layer "B.Cu") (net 6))
 (segment (start 140.5 86) (end 141.75 84.75) (width 0.2) (layer "B.Cu") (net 6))
 (segment (start 141.75 84.75) (end 142.755 84.75) (width 0.2) (layer "B.Cu") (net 6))
 (segment (start 159.31 81.61993) (end 143.92993 97) (width 0.2) (layer "B.Cu") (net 6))
 (segment (start 139.25 78.095) (end 139.25 96.25) (width 0.2) (layer "B.Cu") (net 1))
 (segment (start 139.25 96.25) (end 131.0775 104.4225) (width 0.2) (layer "B.Cu") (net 1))
 (segment (start 131.0775 104.4225) (end 128.455 104.4225) (width 0.2) (layer "B.Cu") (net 1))
 (segment (start 142.755 74.59) (end 139.25 78.095) (width 0.2) (layer "B.Cu") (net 1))
 (segment (start 143.25 105.725) (end 143.25 102.25) (width 0.2) (layer "B.Cu") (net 12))
 (segment (start 163 110) (end 145 110) (width 0.2) (layer "B.Cu") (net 12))
 (segment (start 143.25 108.25) (end 143.25 105.725) (width 0.2) (layer "B.Cu") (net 12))
 (segment (start 141.25 100.25) (end 138.88 100.25) (width 0.2) (layer "B.Cu") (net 12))
 (segment (start 163.85 102.1) (end 163.85 109.15) (width 0.2) (layer "B.Cu") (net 12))
 (segment (start 163.85 109.15) (end 163 110) (width 0.2) (layer "B.Cu") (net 12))
 (segment (start 143.25 102.25) (end 141.25 100.25) (width 0.2) (layer "B.Cu") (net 12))
 (segment (start 145 110) (end 143.25 108.25) (width 0.2) (layer "B.Cu") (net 12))
 (segment (start 161.31 101.145) (end 161.955 100.5) (width 0.2) (layer "B.Cu") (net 13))
 (segment (start 138.036475 99) (end 145.25 99) (width 0.2) (layer "B.Cu") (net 13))
 (segment (start 144 110.5) (end 140.75 107.25) (width 0.2) (layer "B.Cu") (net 13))
 (segment (start 138.725 105.725) (end 137.5 104.5) (width 0.2) (layer "B.Cu") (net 13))
 (segment (start 137.5 99.536475) (end 138.036475 99) (width 0.2) (layer "B.Cu") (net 13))
 (segment (start 137.5 104.5) (end 137.5 99.536475) (width 0.2) (layer "B.Cu") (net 13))
 (segment (start 161.955 100.5) (end 164.5 100.5) (width 0.2) (layer "B.Cu") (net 13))
 (segment (start 145.25 99) (end 146.5 100.25) (width 0.2) (layer "B.Cu") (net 13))
 (segment (start 165.5 109) (end 164 110.5) (width 0.2) (layer "B.Cu") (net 13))
 (segment (start 164.5 100.5) (end 165.5 101.5) (width 0.2) (layer "B.Cu") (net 13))
 (segment (start 164 110.5) (end 144 110.5) (width 0.2) (layer "B.Cu") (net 13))
 (segment (start 161.31 102.1) (end 161.31 101.145) (width 0.2) (layer "B.Cu") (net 13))
 (segment (start 140.75 107.25) (end 140.75 105.725) (width 0.2) (layer "B.Cu") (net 13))
 (segment (start 165.5 101.5) (end 165.5 109) (width 0.2) (layer "B.Cu") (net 13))
 (segment (start 140.75 105.725) (end 138.725 105.725) (width 0.2) (layer "B.Cu") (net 13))
 (segment (start 166.302 101.1678) (end 166.302 109.847) (width 0.2) (layer "B.Cu") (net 14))
 (segment (start 128.149 111.649) (end 124.5 108) (width 0.2) (layer "B.Cu") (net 14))
 (segment (start 124.5 108) (end 124.5 91.575) (width 0.2) (layer "B.Cu") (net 14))
 (segment (start 158.632 99.698) (end 164.8322 99.698) (width 0.2) (layer "B.Cu") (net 14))
 (segment (start 164.5 111.649) (end 128.149 111.649) (width 0.2) (layer "B.Cu") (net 14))
 (segment (start 164.8322 99.698) (end 166.302 101.1678) (width 0.2) (layer "B.Cu") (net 14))
 (segment (start 124.5 91.575) (end 126.245 89.83) (width 0.2) (layer "B.Cu") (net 14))
 (segment (start 156.23 102.1) (end 158.632 99.698) (width 0.2) (layer "B.Cu") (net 14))
 (segment (start 166.302 109.847) (end 164.5 111.649) (width 0.2) (layer "B.Cu") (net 14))
 (segment (start 128.701162 111) (end 125 107.298838) (width 0.2) (layer "B.Cu") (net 15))
 (segment (start 160.771 100.099) (end 164.6661 100.099) (width 0.2) (layer "B.Cu") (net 15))
 (segment (start 165.901 109.599) (end 164.5 111) (width 0.2) (layer "B.Cu") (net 15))
 (segment (start 125 93.615) (end 126.245 92.37) (width 0.2) (layer "B.Cu") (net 15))
 (segment (start 125 107.298838) (end 125 93.615) (width 0.2) (layer "B.Cu") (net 15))
 (segment (start 165.901 101.3339) (end 165.901 109.599) (width 0.2) (layer "B.Cu") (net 15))
 (segment (start 164.5 111) (end 128.701162 111) (width 0.2) (layer "B.Cu") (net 15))
 (segment (start 158.77 102.1) (end 160.771 100.099) (width 0.2) (layer "B.Cu") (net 15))
 (segment (start 164.6661 100.099) (end 165.901 101.3339) (width 0.2) (layer "B.Cu") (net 15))
 (segment (start 165.942 72.942) (end 163.896 70.896) (width 0.2) (layer "B.Cu") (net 4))
 (segment (start 155.619 82.4481) (end 155.619 73.42324) (width 0.2) (layer "B.Cu") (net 4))
 (segment (start 156.29324 72.749) (end 159.78676 72.749) (width 0.2) (layer "B.Cu") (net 4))
 (segment (start 146.5 89.44) (end 148.6271 89.44) (width 0.2) (layer "B.Cu") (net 4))
 (segment (start 144.604 70.896) (end 135.83 79.67) (width 0.2) (layer "B.Cu") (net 4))
 (segment (start 161.77424 75.452) (end 165.03286 75.452) (width 0.2) (layer "B.Cu") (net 4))
 (segment (start 165.942 74.54286) (end 165.942 72.942) (width 0.2) (layer "B.Cu") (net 4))
 (segment (start 160.461 74.13876) (end 161.77424 75.452) (width 0.2) (layer "B.Cu") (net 4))
 (segment (start 159.78676 72.749) (end 160.461 73.42324) (width 0.2) (layer "B.Cu") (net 4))
 (segment (start 165.03286 75.452) (end 165.942 74.54286) (width 0.2) (layer "B.Cu") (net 4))
 (segment (start 155.619 73.42324) (end 156.29324 72.749) (width 0.2) (layer "B.Cu") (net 4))
 (segment (start 148.6271 89.44) (end 155.619 82.4481) (width 0.2) (layer "B.Cu") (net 4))
 (segment (start 135.83 79.67) (end 126.245 79.67) (width 0.2) (layer "B.Cu") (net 4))
 (segment (start 163.896 70.896) (end 144.604 70.896) (width 0.2) (layer "B.Cu") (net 4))
 (segment (start 160.461 73.42324) (end 160.461 74.13876) (width 0.2) (layer "B.Cu") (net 4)))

